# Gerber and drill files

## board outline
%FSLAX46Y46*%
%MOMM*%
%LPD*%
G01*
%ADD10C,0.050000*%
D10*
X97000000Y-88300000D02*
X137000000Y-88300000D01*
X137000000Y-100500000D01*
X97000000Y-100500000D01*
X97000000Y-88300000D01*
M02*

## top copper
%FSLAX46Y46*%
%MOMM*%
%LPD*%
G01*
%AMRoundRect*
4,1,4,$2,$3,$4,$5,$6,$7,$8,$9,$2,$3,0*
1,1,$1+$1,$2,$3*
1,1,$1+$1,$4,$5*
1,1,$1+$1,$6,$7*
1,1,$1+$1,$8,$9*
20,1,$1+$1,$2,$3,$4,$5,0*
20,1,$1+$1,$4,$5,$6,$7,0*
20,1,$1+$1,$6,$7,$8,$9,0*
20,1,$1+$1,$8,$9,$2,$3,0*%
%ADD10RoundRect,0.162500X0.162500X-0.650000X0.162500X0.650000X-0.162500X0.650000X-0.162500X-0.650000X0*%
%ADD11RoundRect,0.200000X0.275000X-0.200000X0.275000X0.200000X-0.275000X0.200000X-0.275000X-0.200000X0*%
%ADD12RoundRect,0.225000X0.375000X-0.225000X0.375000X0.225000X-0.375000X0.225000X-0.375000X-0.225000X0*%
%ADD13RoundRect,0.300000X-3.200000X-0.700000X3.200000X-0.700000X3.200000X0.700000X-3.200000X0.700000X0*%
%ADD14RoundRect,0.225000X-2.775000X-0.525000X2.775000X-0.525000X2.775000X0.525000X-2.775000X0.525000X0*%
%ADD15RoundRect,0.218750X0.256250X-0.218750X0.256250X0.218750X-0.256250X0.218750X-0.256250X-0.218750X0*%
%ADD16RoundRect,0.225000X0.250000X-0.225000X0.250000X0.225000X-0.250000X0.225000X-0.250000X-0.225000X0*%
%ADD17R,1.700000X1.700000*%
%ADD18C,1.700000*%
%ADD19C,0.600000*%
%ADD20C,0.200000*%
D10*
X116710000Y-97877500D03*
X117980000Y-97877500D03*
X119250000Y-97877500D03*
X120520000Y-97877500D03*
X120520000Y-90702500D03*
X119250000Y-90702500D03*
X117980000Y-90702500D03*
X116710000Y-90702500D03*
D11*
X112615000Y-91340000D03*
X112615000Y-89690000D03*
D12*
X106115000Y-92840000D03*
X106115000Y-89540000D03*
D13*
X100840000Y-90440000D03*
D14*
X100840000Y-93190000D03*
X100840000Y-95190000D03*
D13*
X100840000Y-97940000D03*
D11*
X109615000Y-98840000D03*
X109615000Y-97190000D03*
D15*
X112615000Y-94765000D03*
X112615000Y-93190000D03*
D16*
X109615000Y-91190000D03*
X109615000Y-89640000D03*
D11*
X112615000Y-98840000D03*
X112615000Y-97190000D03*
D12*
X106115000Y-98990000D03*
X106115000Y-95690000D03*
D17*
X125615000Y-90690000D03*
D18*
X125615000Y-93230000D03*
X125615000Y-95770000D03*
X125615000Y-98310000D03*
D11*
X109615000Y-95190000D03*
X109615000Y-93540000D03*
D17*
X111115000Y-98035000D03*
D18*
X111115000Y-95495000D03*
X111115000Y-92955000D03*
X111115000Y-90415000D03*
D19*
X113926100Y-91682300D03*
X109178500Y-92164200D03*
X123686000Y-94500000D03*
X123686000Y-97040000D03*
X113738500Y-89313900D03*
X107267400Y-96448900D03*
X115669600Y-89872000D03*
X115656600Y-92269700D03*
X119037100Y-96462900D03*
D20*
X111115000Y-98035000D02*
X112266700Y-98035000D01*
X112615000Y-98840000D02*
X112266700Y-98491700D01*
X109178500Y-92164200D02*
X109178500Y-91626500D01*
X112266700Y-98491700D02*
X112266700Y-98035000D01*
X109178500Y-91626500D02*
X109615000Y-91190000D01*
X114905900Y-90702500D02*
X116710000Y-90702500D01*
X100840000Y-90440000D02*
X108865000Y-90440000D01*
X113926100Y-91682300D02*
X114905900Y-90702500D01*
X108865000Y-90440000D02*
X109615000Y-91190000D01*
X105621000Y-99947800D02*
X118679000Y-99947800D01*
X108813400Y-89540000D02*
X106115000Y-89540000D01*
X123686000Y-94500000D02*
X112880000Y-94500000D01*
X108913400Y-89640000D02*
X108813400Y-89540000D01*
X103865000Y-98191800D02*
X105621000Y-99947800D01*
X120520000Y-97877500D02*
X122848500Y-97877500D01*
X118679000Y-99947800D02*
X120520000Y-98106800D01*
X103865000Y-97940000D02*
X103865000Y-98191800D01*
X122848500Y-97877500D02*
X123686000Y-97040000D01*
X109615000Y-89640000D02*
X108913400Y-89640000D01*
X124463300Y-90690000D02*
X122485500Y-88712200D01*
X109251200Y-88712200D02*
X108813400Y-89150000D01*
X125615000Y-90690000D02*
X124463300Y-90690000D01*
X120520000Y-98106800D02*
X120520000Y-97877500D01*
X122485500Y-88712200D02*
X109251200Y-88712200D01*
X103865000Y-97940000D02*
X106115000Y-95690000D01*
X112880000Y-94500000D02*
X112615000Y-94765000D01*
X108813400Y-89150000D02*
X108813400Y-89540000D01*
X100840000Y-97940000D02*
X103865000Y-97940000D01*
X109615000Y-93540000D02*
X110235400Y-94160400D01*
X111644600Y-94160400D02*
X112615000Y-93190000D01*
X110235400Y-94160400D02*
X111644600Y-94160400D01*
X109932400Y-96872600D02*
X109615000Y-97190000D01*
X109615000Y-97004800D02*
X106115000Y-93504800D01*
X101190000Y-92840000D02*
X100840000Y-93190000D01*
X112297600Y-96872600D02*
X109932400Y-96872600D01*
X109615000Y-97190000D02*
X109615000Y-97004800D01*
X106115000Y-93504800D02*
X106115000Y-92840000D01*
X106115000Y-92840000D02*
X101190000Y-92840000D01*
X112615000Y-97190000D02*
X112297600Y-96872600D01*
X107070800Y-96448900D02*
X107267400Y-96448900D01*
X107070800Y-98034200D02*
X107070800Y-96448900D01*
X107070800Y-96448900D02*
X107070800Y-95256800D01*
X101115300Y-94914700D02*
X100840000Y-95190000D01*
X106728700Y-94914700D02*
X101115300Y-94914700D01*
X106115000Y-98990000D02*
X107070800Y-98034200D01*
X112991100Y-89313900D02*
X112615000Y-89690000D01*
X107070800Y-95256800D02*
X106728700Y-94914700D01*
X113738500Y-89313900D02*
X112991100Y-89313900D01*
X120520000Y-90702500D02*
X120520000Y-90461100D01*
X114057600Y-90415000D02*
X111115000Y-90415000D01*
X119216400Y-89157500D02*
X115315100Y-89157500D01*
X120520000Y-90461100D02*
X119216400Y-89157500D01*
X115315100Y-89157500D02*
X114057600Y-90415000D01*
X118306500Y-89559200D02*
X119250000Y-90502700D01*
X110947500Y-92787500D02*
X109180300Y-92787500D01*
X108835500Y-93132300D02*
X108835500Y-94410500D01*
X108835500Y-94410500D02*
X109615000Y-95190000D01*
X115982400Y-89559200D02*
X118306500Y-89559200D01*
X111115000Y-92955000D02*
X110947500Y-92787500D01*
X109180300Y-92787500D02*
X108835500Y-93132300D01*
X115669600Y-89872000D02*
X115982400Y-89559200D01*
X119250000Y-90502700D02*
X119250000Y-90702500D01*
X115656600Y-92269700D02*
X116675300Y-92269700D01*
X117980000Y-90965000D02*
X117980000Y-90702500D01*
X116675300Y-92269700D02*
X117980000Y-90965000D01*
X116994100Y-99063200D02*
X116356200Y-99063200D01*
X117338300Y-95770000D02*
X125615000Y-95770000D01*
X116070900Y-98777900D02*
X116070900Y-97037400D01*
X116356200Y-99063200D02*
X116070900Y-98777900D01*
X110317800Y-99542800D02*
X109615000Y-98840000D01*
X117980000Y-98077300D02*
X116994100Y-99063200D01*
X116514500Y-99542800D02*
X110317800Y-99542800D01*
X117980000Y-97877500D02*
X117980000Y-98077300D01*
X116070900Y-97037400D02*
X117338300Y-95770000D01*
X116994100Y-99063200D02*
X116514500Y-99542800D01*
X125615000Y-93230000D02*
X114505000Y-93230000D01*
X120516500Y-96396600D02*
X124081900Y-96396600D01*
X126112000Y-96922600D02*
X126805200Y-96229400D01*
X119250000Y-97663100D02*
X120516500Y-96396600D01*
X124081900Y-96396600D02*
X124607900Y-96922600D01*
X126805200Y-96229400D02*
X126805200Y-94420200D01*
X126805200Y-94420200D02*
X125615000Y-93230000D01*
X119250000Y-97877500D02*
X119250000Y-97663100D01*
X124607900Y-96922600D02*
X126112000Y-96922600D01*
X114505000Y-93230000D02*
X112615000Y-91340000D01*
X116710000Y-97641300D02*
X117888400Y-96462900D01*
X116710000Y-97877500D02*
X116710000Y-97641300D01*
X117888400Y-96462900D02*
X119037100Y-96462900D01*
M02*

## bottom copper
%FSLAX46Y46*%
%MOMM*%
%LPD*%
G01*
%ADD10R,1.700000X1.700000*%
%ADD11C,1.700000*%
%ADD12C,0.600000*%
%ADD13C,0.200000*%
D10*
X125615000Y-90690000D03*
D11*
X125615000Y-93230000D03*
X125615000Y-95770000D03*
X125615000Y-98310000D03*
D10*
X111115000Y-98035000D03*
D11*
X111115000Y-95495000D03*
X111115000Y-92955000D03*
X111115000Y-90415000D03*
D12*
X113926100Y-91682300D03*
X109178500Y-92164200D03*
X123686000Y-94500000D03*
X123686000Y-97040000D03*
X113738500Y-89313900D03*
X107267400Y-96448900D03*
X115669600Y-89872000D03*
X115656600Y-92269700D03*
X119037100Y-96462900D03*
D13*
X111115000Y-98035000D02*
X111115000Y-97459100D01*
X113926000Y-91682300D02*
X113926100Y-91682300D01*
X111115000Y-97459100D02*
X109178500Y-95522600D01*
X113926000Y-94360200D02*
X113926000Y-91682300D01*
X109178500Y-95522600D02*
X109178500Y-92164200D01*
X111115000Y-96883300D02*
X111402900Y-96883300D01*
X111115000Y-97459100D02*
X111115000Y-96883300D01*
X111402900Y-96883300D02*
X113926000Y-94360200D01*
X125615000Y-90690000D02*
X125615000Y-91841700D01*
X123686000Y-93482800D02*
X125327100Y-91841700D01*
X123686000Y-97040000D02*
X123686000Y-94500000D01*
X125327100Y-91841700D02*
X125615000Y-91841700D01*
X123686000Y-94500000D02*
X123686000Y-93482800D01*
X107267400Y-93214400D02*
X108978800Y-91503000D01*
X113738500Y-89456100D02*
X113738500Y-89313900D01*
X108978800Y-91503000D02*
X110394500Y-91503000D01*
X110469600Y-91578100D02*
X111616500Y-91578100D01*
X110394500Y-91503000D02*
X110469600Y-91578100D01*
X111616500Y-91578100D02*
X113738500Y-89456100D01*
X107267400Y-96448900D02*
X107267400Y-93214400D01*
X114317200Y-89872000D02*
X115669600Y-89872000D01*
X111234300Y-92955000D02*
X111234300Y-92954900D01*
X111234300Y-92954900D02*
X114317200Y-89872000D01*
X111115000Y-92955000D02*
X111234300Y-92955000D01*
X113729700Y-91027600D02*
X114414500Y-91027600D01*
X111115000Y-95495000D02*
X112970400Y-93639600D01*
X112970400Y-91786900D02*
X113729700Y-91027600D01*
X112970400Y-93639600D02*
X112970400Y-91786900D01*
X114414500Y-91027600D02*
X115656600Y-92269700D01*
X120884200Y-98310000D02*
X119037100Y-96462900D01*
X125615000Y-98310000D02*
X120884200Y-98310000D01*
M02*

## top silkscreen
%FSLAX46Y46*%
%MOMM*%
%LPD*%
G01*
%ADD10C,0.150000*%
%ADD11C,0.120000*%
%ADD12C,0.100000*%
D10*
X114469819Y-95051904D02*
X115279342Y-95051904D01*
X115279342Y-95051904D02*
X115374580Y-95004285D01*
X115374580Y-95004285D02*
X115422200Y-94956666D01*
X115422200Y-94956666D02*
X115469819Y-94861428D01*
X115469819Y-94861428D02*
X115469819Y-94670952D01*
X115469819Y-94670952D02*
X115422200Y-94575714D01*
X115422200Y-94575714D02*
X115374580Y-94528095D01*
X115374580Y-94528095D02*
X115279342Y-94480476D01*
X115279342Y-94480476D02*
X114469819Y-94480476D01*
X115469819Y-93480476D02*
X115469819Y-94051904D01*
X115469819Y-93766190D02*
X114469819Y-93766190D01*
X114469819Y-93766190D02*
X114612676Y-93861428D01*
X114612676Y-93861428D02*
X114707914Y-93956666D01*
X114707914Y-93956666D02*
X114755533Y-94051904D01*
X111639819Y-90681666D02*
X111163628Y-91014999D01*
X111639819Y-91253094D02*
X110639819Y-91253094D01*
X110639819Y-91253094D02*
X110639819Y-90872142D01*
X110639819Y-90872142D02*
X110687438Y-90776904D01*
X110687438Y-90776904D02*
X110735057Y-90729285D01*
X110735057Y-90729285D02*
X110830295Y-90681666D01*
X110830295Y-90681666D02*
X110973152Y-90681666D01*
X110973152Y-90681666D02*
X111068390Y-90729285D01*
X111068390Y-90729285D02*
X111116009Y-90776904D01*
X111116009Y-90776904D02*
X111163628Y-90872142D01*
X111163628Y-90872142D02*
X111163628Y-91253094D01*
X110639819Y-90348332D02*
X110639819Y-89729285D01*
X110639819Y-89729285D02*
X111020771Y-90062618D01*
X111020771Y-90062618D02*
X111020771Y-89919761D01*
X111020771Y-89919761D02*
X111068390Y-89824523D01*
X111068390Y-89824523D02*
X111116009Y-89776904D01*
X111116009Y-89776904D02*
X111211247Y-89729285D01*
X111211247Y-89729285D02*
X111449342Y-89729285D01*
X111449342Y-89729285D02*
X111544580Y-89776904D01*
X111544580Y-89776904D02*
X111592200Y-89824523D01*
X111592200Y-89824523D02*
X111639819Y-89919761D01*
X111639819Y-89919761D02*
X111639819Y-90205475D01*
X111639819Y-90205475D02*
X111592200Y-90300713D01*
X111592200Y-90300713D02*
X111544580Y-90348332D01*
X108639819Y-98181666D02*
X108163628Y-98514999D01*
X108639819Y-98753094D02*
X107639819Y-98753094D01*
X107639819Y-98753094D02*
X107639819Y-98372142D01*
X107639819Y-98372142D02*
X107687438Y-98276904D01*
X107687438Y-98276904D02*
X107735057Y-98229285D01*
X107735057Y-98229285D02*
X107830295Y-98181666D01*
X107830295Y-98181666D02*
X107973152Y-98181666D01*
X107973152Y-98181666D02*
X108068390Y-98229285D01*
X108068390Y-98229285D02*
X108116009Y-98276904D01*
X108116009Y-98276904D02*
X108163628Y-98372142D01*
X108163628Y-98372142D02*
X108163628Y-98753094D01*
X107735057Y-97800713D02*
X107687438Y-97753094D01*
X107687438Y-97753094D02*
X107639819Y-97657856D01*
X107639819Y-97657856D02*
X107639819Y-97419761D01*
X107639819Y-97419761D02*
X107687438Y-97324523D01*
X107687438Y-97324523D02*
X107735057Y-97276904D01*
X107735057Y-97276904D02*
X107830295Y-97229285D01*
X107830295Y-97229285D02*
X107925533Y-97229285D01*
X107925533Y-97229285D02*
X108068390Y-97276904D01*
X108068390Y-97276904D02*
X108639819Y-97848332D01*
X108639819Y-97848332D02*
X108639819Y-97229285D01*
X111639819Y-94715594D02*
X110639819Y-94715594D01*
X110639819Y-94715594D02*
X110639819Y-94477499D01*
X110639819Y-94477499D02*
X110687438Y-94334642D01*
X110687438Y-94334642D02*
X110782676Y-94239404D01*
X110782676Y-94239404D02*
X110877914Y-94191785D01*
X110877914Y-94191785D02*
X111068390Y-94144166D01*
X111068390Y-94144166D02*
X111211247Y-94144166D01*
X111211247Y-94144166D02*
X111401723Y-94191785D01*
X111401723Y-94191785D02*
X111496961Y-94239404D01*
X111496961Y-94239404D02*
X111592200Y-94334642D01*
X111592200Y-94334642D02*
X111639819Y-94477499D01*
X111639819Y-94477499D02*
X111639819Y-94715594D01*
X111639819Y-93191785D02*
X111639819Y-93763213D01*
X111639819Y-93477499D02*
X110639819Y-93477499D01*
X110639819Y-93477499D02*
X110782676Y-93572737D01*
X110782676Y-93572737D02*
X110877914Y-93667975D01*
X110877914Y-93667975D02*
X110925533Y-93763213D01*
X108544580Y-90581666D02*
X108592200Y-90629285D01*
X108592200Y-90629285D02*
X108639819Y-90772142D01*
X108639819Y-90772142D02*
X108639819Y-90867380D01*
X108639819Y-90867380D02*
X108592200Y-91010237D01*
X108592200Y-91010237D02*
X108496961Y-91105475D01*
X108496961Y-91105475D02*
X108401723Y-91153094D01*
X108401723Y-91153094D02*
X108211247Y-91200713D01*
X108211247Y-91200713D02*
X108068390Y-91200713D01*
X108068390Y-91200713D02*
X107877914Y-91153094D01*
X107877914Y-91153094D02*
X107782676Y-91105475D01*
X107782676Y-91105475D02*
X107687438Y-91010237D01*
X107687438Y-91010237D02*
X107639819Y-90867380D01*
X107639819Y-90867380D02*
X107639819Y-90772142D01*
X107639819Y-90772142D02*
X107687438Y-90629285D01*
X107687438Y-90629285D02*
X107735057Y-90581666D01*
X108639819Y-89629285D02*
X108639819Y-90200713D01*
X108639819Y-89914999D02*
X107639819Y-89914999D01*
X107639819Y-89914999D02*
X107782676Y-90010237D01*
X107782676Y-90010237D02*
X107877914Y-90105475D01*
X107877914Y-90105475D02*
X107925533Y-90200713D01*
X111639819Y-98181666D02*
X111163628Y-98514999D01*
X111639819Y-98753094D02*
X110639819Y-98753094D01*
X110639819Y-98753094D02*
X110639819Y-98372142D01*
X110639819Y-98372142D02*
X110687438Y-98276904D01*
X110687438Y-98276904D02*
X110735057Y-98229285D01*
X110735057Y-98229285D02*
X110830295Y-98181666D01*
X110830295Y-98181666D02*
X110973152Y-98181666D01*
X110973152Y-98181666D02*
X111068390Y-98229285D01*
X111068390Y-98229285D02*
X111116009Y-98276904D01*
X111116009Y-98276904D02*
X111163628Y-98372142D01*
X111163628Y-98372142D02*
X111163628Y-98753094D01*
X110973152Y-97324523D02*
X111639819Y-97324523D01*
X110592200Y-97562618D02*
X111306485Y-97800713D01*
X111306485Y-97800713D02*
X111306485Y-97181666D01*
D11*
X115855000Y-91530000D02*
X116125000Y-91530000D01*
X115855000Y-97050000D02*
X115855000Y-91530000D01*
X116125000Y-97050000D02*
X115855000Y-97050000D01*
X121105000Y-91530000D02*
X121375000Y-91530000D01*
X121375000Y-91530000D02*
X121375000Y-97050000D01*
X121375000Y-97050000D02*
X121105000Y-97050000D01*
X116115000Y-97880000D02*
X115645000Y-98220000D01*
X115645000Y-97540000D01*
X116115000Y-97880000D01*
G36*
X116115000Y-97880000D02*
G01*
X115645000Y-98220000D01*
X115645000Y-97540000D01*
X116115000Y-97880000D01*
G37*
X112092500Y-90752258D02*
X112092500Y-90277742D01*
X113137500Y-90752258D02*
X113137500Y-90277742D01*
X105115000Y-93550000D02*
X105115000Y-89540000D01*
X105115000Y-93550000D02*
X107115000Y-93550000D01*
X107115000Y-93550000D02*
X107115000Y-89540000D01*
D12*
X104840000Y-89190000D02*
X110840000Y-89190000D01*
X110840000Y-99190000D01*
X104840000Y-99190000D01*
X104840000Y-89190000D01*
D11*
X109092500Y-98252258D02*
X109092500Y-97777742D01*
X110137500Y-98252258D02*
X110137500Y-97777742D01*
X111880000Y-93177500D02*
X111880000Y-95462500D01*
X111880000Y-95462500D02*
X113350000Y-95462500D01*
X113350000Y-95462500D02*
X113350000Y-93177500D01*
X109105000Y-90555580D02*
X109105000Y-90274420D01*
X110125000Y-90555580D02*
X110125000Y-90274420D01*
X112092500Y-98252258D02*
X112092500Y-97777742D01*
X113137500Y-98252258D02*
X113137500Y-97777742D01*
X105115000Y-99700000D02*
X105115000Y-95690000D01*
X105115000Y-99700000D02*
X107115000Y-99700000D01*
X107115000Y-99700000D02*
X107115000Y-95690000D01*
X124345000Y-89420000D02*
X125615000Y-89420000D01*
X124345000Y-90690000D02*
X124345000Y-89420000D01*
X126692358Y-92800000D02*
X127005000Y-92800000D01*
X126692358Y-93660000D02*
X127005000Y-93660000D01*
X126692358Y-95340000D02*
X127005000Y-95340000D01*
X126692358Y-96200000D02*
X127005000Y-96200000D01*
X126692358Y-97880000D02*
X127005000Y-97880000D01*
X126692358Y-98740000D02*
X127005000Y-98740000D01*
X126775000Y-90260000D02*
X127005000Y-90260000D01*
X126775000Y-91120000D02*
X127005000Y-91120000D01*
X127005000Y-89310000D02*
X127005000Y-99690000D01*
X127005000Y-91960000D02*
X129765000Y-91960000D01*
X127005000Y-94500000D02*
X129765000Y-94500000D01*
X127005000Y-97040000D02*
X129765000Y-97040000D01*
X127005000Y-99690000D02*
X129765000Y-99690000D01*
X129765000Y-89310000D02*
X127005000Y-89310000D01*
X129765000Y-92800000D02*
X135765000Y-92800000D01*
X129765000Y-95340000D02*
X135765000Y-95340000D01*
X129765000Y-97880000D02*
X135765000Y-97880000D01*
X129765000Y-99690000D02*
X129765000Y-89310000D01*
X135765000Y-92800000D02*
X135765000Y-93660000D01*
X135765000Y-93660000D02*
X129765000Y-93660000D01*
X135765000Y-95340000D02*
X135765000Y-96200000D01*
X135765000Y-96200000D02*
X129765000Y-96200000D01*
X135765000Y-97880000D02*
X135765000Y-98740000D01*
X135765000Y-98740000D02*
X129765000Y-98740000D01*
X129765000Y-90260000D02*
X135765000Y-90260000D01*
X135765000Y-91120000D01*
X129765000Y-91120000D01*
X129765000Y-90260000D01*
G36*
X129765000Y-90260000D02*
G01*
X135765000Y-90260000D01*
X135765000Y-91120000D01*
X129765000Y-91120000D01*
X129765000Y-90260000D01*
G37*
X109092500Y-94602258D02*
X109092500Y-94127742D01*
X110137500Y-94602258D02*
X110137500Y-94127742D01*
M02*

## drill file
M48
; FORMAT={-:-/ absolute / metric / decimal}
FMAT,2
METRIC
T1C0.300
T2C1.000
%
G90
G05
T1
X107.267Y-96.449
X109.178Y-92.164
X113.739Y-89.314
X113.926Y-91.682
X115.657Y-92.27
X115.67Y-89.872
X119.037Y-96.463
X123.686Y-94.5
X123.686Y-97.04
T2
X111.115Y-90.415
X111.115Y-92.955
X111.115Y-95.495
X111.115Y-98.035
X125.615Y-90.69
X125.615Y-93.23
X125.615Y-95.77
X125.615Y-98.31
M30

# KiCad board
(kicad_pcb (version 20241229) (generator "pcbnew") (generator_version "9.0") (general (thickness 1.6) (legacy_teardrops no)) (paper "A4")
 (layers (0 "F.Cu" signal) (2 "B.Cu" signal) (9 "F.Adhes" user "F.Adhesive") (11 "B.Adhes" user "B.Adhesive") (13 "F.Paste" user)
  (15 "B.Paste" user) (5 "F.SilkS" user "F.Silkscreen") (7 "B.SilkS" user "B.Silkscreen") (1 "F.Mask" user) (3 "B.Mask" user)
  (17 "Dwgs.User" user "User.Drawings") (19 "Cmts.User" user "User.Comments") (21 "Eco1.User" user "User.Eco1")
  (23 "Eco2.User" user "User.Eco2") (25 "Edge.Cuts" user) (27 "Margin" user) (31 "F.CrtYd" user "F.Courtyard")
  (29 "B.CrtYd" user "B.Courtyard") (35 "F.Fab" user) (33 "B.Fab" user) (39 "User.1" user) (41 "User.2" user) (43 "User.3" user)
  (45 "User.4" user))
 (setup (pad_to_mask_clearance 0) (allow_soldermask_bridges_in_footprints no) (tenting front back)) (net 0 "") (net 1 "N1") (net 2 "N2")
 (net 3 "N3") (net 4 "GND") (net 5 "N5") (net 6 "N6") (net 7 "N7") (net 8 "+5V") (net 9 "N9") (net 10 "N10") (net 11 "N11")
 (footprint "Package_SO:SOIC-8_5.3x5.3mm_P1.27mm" (layer "F.Cu") (at 118.615 94.29 90)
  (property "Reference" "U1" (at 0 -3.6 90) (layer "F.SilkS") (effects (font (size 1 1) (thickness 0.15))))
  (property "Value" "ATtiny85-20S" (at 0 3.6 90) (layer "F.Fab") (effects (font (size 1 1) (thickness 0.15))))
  (fp_line (start 2.76 -2.76) (end 2.76 -2.49) (stroke (width 0.12) (type solid)) (layer "F.SilkS"))
  (fp_line (start -2.76 -2.76) (end 2.76 -2.76) (stroke (width 0.12) (type solid)) (layer "F.SilkS"))
  (fp_line (start -2.76 -2.49) (end -2.76 -2.76) (stroke (width 0.12) (type solid)) (layer "F.SilkS"))
  (fp_line (start 2.76 2.49) (end 2.76 2.76) (stroke (width 0.12) (type solid)) (layer "F.SilkS"))
  (fp_line (start 2.76 2.76) (end -2.76 2.76) (stroke (width 0.12) (type solid)) (layer "F.SilkS"))
  (fp_line (start -2.76 2.76) (end -2.76 2.49) (stroke (width 0.12) (type solid)) (layer "F.SilkS"))
  (fp_poly (pts (xy -3.59 -2.5) (xy -3.93 -2.97) (xy -3.25 -2.97)) (stroke (width 0.12) (type solid)) (fill yes) (layer "F.SilkS"))
  (pad "1" smd roundrect (at -3.5875 -1.905 90) (size 1.625 0.65) (layers "F.Cu" "F.Mask" "F.Paste") (roundrect_rratio 0.25) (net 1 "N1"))
  (pad "2" smd roundrect (at -3.5875 -0.635 90) (size 1.625 0.65) (layers "F.Cu" "F.Mask" "F.Paste") (roundrect_rratio 0.25) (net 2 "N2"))
  (pad "3" smd roundrect (at -3.5875 0.635 90) (size 1.625 0.65) (layers "F.Cu" "F.Mask" "F.Paste") (roundrect_rratio 0.25) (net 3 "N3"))
  (pad "4" smd roundrect (at -3.5875 1.905 90) (size 1.625 0.65) (layers "F.Cu" "F.Mask" "F.Paste") (roundrect_rratio 0.25) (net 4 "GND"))
  (pad "5" smd roundrect (at 3.5875 1.905 90) (size 1.625 0.65) (layers "F.Cu" "F.Mask" "F.Paste") (roundrect_rratio 0.25) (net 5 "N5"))
  (pad "6" smd roundrect (at 3.5875 0.635 90) (size 1.625 0.65) (layers "F.Cu" "F.Mask" "F.Paste") (roundrect_rratio 0.25) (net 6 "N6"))
  (pad "7" smd roundrect (at 3.5875 -0.635 90) (size 1.625 0.65) (layers "F.Cu" "F.Mask" "F.Paste") (roundrect_rratio 0.25) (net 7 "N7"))
  (pad "8" smd roundrect (at 3.5875 -1.905 90) (size 1.625 0.65) (layers "F.Cu" "F.Mask" "F.Paste") (roundrect_rratio 0.25) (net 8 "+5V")))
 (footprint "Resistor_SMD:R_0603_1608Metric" (layer "F.Cu") (at 112.615 90.515 90)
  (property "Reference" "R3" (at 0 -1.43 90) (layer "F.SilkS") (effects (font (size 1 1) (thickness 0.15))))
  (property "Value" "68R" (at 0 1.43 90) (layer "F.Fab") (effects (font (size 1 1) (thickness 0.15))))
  (fp_line (start -0.237258 -0.5225) (end 0.237258 -0.5225) (stroke (width 0.12) (type solid)) (layer "F.SilkS"))
  (fp_line (start -0.237258 0.5225) (end 0.237258 0.5225) (stroke (width 0.12) (type solid)) (layer "F.SilkS"))
  (pad "1" smd roundrect (at -0.825 0 90) (size 0.8 0.95) (layers "F.Cu" "F.Mask" "F.Paste") (roundrect_rratio 0.25) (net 3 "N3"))
  (pad "2" smd roundrect (at 0.825 0 90) (size 0.8 0.95) (layers "F.Cu" "F.Mask" "F.Paste") (roundrect_rratio 0.25) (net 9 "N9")))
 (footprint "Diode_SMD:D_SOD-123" (layer "F.Cu") (at 106.115 91.19 90)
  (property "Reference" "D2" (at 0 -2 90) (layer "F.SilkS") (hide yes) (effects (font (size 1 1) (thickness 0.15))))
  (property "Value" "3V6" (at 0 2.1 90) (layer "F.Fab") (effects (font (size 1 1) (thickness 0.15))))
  (fp_line (start -2.36 -1) (end 1.65 -1) (stroke (width 0.12) (type solid)) (layer "F.SilkS"))
  (fp_line (start -2.36 -1) (end -2.36 1) (stroke (width 0.12) (type solid)) (layer "F.SilkS"))
  (fp_line (start -2.36 1) (end 1.65 1) (stroke (width 0.12) (type solid)) (layer "F.SilkS"))
  (pad "1" smd roundrect (at -1.65 0 90) (size 0.9 1.2) (layers "F.Cu" "F.Mask" "F.Paste") (roundrect_rratio 0.25) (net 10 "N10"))
  (pad "2" smd roundrect (at 1.65 0 90) (size 0.9 1.2) (layers "F.Cu" "F.Mask" "F.Paste") (roundrect_rratio 0.25) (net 4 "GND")))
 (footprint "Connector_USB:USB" (layer "F.Cu") (at 100.84 94.19)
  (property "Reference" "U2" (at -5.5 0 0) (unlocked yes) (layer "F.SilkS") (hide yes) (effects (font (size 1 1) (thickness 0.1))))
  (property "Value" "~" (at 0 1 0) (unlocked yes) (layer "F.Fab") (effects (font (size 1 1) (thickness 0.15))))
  (fp_rect (start 4 -5) (end 10 5) (stroke (width 0.1) (type default)) (fill no) (layer "F.SilkS"))
  (pad "1" smd roundrect (at 0 -3.75) (size 7 2) (layers "F.Cu" "F.Mask" "F.Paste") (roundrect_rratio 0.15) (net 8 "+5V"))
  (pad "2" smd roundrect (at 0 -1) (size 6 1.5) (layers "F.Cu" "F.Mask" "F.Paste") (roundrect_rratio 0.15) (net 10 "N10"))
  (pad "3" smd roundrect (at 0 1) (size 6 1.5) (layers "F.Cu" "F.Mask" "F.Paste") (roundrect_rratio 0.15) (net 9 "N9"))
  (pad "4" smd roundrect (at 0 3.75) (size 7 2) (layers "F.Cu" "F.Mask" "F.Paste") (roundrect_rratio 0.15) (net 4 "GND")))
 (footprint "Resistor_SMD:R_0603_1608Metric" (layer "F.Cu") (at 109.615 98.015 90)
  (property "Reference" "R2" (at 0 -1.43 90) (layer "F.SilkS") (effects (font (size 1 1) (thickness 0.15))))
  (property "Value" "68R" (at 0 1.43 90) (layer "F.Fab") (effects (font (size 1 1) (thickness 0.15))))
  (fp_line (start -0.237258 -0.5225) (end 0.237258 -0.5225) (stroke (width 0.12) (type solid)) (layer "F.SilkS"))
  (fp_line (start -0.237258 0.5225) (end 0.237258 0.5225) (stroke (width 0.12) (type solid)) (layer "F.SilkS"))
  (pad "1" smd roundrect (at -0.825 0 90) (size 0.8 0.95) (layers "F.Cu" "F.Mask" "F.Paste") (roundrect_rratio 0.25) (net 2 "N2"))
  (pad "2" smd roundrect (at 0.825 0 90) (size 0.8 0.95) (layers "F.Cu" "F.Mask" "F.Paste") (roundrect_rratio 0.25) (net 10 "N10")))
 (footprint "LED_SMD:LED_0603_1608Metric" (layer "F.Cu") (at 112.615 93.9775 90)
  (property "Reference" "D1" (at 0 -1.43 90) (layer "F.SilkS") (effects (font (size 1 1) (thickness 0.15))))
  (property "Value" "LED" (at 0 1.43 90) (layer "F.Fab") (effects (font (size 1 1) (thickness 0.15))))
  (fp_line (start 0.8 -0.735) (end -1.485 -0.735) (stroke (width 0.12) (type solid)) (layer "F.SilkS"))
  (fp_line (start -1.485 -0.735) (end -1.485 0.735) (stroke (width 0.12) (type solid)) (layer "F.SilkS"))
  (fp_line (start -1.485 0.735) (end 0.8 0.735) (stroke (width 0.12) (type solid)) (layer "F.SilkS"))
  (pad "1" smd roundrect (at -0.7875 0 90) (size 0.875 0.95) (layers "F.Cu" "F.Mask" "F.Paste") (roundrect_rratio 0.25) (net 4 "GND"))
  (pad "2" smd roundrect (at 0.7875 0 90) (size 0.875 0.95) (layers "F.Cu" "F.Mask" "F.Paste") (roundrect_rratio 0.25) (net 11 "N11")))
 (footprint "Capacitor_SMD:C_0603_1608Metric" (layer "F.Cu") (at 109.615 90.415 90)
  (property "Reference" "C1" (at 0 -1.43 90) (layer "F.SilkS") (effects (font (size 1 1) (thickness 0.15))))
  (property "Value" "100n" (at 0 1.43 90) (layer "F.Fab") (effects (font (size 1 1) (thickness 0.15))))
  (fp_line (start -0.14058 -0.51) (end 0.14058 -0.51) (stroke (width 0.12) (type solid)) (layer "F.SilkS"))
  (fp_line (start -0.14058 0.51) (end 0.14058 0.51) (stroke (width 0.12) (type solid)) (layer "F.SilkS"))
  (pad "1" smd roundrect (at -0.775 0 90) (size 0.9 0.95) (layers "F.Cu" "F.Mask" "F.Paste") (roundrect_rratio 0.25) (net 8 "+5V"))
  (pad "2" smd roundrect (at 0.775 0 90) (size 0.9 0.95) (layers "F.Cu" "F.Mask" "F.Paste") (roundrect_rratio 0.25) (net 4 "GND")))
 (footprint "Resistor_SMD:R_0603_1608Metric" (layer "F.Cu") (at 112.615 98.015 90)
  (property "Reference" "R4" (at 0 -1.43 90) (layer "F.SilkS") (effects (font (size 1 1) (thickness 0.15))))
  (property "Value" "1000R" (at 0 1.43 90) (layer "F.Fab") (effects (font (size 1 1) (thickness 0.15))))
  (fp_line (start -0.237258 -0.5225) (end 0.237258 -0.5225) (stroke (width 0.12) (type solid)) (layer "F.SilkS"))
  (fp_line (start -0.237258 0.5225) (end 0.237258 0.5225) (stroke (width 0.12) (type solid)) (layer "F.SilkS"))
  (pad "1" smd roundrect (at -0.825 0 90) (size 0.8 0.95) (layers "F.Cu" "F.Mask" "F.Paste") (roundrect_rratio 0.25) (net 8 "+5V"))
  (pad "2" smd roundrect (at 0.825 0 90) (size 0.8 0.95) (layers "F.Cu" "F.Mask" "F.Paste") (roundrect_rratio 0.25) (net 10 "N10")))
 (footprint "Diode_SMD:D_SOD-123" (layer "F.Cu") (at 106.115 97.34 90)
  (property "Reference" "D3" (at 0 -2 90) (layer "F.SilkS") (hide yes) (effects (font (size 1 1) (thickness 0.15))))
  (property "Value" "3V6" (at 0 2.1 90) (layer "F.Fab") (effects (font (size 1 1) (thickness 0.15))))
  (fp_line (start -2.36 -1) (end 1.65 -1) (stroke (width 0.12) (type solid)) (layer "F.SilkS"))
  (fp_line (start -2.36 -1) (end -2.36 1) (stroke (width 0.12) (type solid)) (layer "F.SilkS"))
  (fp_line (start -2.36 1) (end 1.65 1) (stroke (width 0.12) (type solid)) (layer "F.SilkS"))
  (pad "1" smd roundrect (at -1.65 0 90) (size 0.9 1.2) (layers "F.Cu" "F.Mask" "F.Paste") (roundrect_rratio 0.25) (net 9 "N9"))
  (pad "2" smd roundrect (at 1.65 0 90) (size 0.9 1.2) (layers "F.Cu" "F.Mask" "F.Paste") (roundrect_rratio 0.25) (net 4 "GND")))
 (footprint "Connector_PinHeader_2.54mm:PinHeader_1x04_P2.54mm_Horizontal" (layer "F.Cu") (at 125.615 90.69)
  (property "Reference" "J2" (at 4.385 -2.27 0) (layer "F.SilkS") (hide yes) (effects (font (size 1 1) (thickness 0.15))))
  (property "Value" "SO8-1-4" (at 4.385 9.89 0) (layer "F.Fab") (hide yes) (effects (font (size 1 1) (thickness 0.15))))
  (fp_line (start -1.27 -1.27) (end 0 -1.27) (stroke (width 0.12) (type solid)) (layer "F.SilkS"))
  (fp_line (start -1.27 0) (end -1.27 -1.27) (stroke (width 0.12) (type solid)) (layer "F.SilkS"))
  (fp_line (start 1.077358 2.11) (end 1.39 2.11) (stroke (width 0.12) (type solid)) (layer "F.SilkS"))
  (fp_line (start 1.077358 2.97) (end 1.39 2.97) (stroke (width 0.12) (type solid)) (layer "F.SilkS"))
  (fp_line (start 1.077358 4.65) (end 1.39 4.65) (stroke (width 0.12) (type solid)) (layer "F.SilkS"))
  (fp_line (start 1.077358 5.51) (end 1.39 5.51) (stroke (width 0.12) (type solid)) (layer "F.SilkS"))
  (fp_line (start 1.077358 7.19) (end 1.39 7.19) (stroke (width 0.12) (type solid)) (layer "F.SilkS"))
  (fp_line (start 1.077358 8.05) (end 1.39 8.05) (stroke (width 0.12) (type solid)) (layer "F.SilkS"))
  (fp_line (start 1.16 -0.43) (end 1.39 -0.43) (stroke (width 0.12) (type solid)) (layer "F.SilkS"))
  (fp_line (start 1.16 0.43) (end 1.39 0.43) (stroke (width 0.12) (type solid)) (layer "F.SilkS"))
  (fp_line (start 1.39 -1.38) (end 1.39 9) (stroke (width 0.12) (type solid)) (layer "F.SilkS"))
  (fp_line (start 1.39 1.27) (end 4.15 1.27) (stroke (width 0.12) (type solid)) (layer "F.SilkS"))
  (fp_line (start 1.39 3.81) (end 4.15 3.81) (stroke (width 0.12) (type solid)) (layer "F.SilkS"))
  (fp_line (start 1.39 6.35) (end 4.15 6.35) (stroke (width 0.12) (type solid)) (layer "F.SilkS"))
  (fp_line (start 1.39 9) (end 4.15 9) (stroke (width 0.12) (type solid)) (layer "F.SilkS"))
  (fp_line (start 4.15 -1.38) (end 1.39 -1.38) (stroke (width 0.12) (type solid)) (layer "F.SilkS"))
  (fp_line (start 4.15 2.11) (end 10.15 2.11) (stroke (width 0.12) (type solid)) (layer "F.SilkS"))
  (fp_line (start 4.15 4.65) (end 10.15 4.65) (stroke (width 0.12) (type solid)) (layer "F.SilkS"))
  (fp_line (start 4.15 7.19) (end 10.15 7.19) (stroke (width 0.12) (type solid)) (layer "F.SilkS"))
  (fp_line (start 4.15 9) (end 4.15 -1.38) (stroke (width 0.12) (type solid)) (layer "F.SilkS"))
  (fp_line (start 10.15 2.11) (end 10.15 2.97) (stroke (width 0.12) (type solid)) (layer "F.SilkS"))
  (fp_line (start 10.15 2.97) (end 4.15 2.97) (stroke (width 0.12) (type solid)) (layer "F.SilkS"))
  (fp_line (start 10.15 4.65) (end 10.15 5.51) (stroke (width 0.12) (type solid)) (layer "F.SilkS"))
  (fp_line (start 10.15 5.51) (end 4.15 5.51) (stroke (width 0.12) (type solid)) (layer "F.SilkS"))
  (fp_line (start 10.15 7.19) (end 10.15 8.05) (stroke (width 0.12) (type solid)) (layer "F.SilkS"))
  (fp_line (start 10.15 8.05) (end 4.15 8.05) (stroke (width 0.12) (type solid)) (layer "F.SilkS"))
  (fp_rect (start 4.15 -0.43) (end 10.15 0.43) (stroke (width 0.12) (type solid)) (fill yes) (layer "F.SilkS"))
  (pad "1" thru_hole rect (at 0 0) (size 1.7 1.7) (drill 1) (layers "*.Cu" "*.Mask") (remove_unused_layers no) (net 4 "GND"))
  (pad "2" thru_hole circle (at 0 2.54) (size 1.7 1.7) (drill 1) (layers "*.Cu" "*.Mask") (remove_unused_layers no) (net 3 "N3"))
  (pad "3" thru_hole circle (at 0 5.08) (size 1.7 1.7) (drill 1) (layers "*.Cu" "*.Mask") (remove_unused_layers no) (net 2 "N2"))
  (pad "4" thru_hole circle (at 0 7.62) (size 1.7 1.7) (drill 1) (layers "*.Cu" "*.Mask") (remove_unused_layers no) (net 1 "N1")))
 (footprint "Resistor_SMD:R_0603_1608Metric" (layer "F.Cu") (at 109.615 94.365 90)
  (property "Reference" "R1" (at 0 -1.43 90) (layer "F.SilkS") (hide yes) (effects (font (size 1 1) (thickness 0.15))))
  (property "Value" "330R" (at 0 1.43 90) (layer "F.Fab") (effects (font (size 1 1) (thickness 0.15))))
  (fp_line (start -0.237258 -0.5225) (end 0.237258 -0.5225) (stroke (width 0.12) (type solid)) (layer "F.SilkS"))
  (fp_line (start -0.237258 0.5225) (end 0.237258 0.5225) (stroke (width 0.12) (type solid)) (layer "F.SilkS"))
  (pad "1" smd roundrect (at -0.825 0 90) (size 0.8 0.95) (layers "F.Cu" "F.Mask" "F.Paste") (roundrect_rratio 0.25) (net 6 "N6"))
  (pad "2" smd roundrect (at 0.825 0 90) (size 0.8 0.95) (layers "F.Cu" "F.Mask" "F.Paste") (roundrect_rratio 0.25) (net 11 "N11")))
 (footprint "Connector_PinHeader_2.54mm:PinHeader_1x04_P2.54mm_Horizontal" (layer "B.Cu") (at 111.115 98.035)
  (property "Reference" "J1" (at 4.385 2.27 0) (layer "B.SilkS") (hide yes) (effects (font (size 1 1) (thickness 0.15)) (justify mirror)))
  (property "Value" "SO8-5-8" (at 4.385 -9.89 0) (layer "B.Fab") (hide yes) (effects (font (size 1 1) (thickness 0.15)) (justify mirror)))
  (pad "1" thru_hole rect (at 0 0) (size 1.7 1.7) (drill 1) (layers "*.Cu" "*.Mask") (remove_unused_layers no) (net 8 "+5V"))
  (pad "2" thru_hole circle (at 0 -2.54) (size 1.7 1.7) (drill 1) (layers "*.Cu" "*.Mask") (remove_unused_layers no) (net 7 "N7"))
  (pad "3" thru_hole circle (at 0 -5.08) (size 1.7 1.7) (drill 1) (layers "*.Cu" "*.Mask") (remove_unused_layers no) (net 6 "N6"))
  (pad "4" thru_hole circle (at 0 -7.62) (size 1.7 1.7) (drill 1) (layers "*.Cu" "*.Mask") (remove_unused_layers no) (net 5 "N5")))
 (gr_rect (start 97 88.3) (end 137 100.5) (stroke (width 0.05) (type solid)) (fill no) (layer "Edge.Cuts"))
 (segment (start 111.115 98.035) (end 112.2667 98.035) (width 0.2) (layer "F.Cu") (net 8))
 (segment (start 112.615 98.84) (end 112.2667 98.4917) (width 0.2) (layer "F.Cu") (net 8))
 (segment (start 109.1785 92.1642) (end 109.1785 91.6265) (width 0.2) (layer "F.Cu") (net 8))
 (segment (start 112.2667 98.4917) (end 112.2667 98.035) (width 0.2) (layer "F.Cu") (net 8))
 (segment (start 109.1785 91.6265) (end 109.615 91.19) (width 0.2) (layer "F.Cu") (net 8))
 (segment (start 114.9059 90.7025) (end 116.71 90.7025) (width 0.2) (layer "F.Cu") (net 8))
 (segment (start 100.84 90.44) (end 108.865 90.44) (width 0.2) (layer "F.Cu") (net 8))
 (segment (start 113.9261 91.6823) (end 114.9059 90.7025) (width 0.2) (layer "F.Cu") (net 8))
 (segment (start 108.865 90.44) (end 109.615 91.19) (width 0.2) (layer "F.Cu") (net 8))
 (via (at 113.9261 91.6823) (size 0.6) (drill 0.3) (layers "F.Cu" "B.Cu") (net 8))
 (via (at 109.1785 92.1642) (size 0.6) (drill 0.3) (layers "F.Cu" "B.Cu") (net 8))
 (segment (start 111.115 98.035) (end 111.115 97.4591) (width 0.2) (layer "B.Cu") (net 8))
 (segment (start 113.926 91.6823) (end 113.9261 91.6823) (width 0.2) (layer "B.Cu") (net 8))
 (segment (start 111.115 97.4591) (end 109.1785 95.5226) (width 0.2) (layer "B.Cu") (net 8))
 (segment (start 113.926 94.3602) (end 113.926 91.6823) (width 0.2) (layer "B.Cu") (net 8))
 (segment (start 109.1785 95.5226) (end 109.1785 92.1642) (width 0.2) (layer "B.Cu") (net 8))
 (segment (start 111.115 96.8833) (end 111.4029 96.8833) (width 0.2) (layer "B.Cu") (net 8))
 (segment (start 111.115 97.4591) (end 111.115 96.8833) (width 0.2) (layer "B.Cu") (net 8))
 (segment (start 111.4029 96.8833) (end 113.926 94.3602) (width 0.2) (layer "B.Cu") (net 8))
 (segment (start 105.621 99.9478) (end 118.679 99.9478) (width 0.2) (layer "F.Cu") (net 4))
 (segment (start 108.8134 89.54) (end 106.115 89.54) (width 0.2) (layer "F.Cu") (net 4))
 (segment (start 123.686 94.5) (end 112.88 94.5) (width 0.2) (layer "F.Cu") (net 4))
 (segment (start 108.9134 89.64) (end 108.8134 89.54) (width 0.2) (layer "F.Cu") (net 4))
 (segment (start 103.865 98.1918) (end 105.621 99.9478) (width 0.2) (layer "F.Cu") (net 4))
 (segment (start 120.52 97.8775) (end 122.8485 97.8775) (width 0.2) (layer "F.Cu") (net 4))
 (segment (start 118.679 99.9478) (end 120.52 98.1068) (width 0.2) (layer "F.Cu") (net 4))
 (segment (start 103.865 97.94) (end 103.865 98.1918) (width 0.2) (layer "F.Cu") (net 4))
 (segment (start 122.8485 97.8775) (end 123.686 97.04) (width 0.2) (layer "F.Cu") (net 4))
 (segment (start 109.615 89.64) (end 108.9134 89.64) (width 0.2) (layer "F.Cu") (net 4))
 (segment (start 124.4633 90.69) (end 122.4855 88.7122) (width 0.2) (layer "F.Cu") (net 4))
 (segment (start 109.2512 88.7122) (end 108.8134 89.15) (width 0.2) (layer "F.Cu") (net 4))
 (segment (start 125.615 90.69) (end 124.4633 90.69) (width 0.2) (layer "F.Cu") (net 4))
 (segment (start 120.52 98.1068) (end 120.52 97.8775) (width 0.2) (layer "F.Cu") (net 4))
 (segment (start 122.4855 88.7122) (end 109.2512 88.7122) (width 0.2) (layer "F.Cu") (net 4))
 (segment (start 103.865 97.94) (end 106.115 95.69) (width 0.2) (layer "F.Cu") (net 4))
 (segment (start 112.88 94.5) (end 112.615 94.765) (width 0.2) (layer "F.Cu") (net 4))
 (segment (start 108.8134 89.15) (end 108.8134 89.54) (width 0.2) (layer "F.Cu") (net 4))
 (segment (start 100.84 97.94) (end 103.865 97.94) (width 0.2) (layer "F.Cu") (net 4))
 (via (at 123.686 94.5) (size 0.6) (drill 0.3) (layers "F.Cu" "B.Cu") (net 4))
 (via (at 123.686 97.04) (size 0.6) (drill 0.3) (layers "F.Cu" "B.Cu") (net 4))
 (segment (start 125.615 90.69) (end 125.615 91.8417) (width 0.2) (layer "B.Cu") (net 4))
 (segment (start 123.686 93.4828) (end 125.3271 91.8417) (width 0.2) (layer "B.Cu") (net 4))
 (segment (start 123.686 97.04) (end 123.686 94.5) (width 0.2) (layer "B.Cu") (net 4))
 (segment (start 125.3271 91.8417) (end 125.615 91.8417) (width 0.2) (layer "B.Cu") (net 4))
 (segment (start 123.686 94.5) (end 123.686 93.4828) (width 0.2) (layer "B.Cu") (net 4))
 (segment (start 109.615 93.54) (end 110.2354 94.1604) (width 0.2) (layer "F.Cu") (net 11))
 (segment (start 111.6446 94.1604) (end 112.615 93.19) (width 0.2) (layer "F.Cu") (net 11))
 (segment (start 110.2354 94.1604) (end 111.6446 94.1604) (width 0.2) (layer "F.Cu") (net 11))
 (segment (start 109.9324 96.8726) (end 109.615 97.19) (width 0.2) (layer "F.Cu") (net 10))
 (segment (start 109.615 97.0048) (end 106.115 93.5048) (width 0.2) (layer "F.Cu") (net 10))
 (segment (start 101.19 92.84) (end 100.84 93.19) (width 0.2) (layer "F.Cu") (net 10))
 (segment (start 112.2976 96.8726) (end 109.9324 96.8726) (width 0.2) (layer "F.Cu") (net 10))
 (segment (start 109.615 97.19) (end 109.615 97.0048) (width 0.2) (layer "F.Cu") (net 10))
 (segment (start 106.115 93.5048) (end 106.115 92.84) (width 0.2) (layer "F.Cu") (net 10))
 (segment (start 106.115 92.84) (end 101.19 92.84) (width 0.2) (layer "F.Cu") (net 10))
 (segment (start 112.615 97.19) (end 112.2976 96.8726) (width 0.2) (layer "F.Cu") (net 10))
 (segment (start 107.0708 96.4489) (end 107.2674 96.4489) (width 0.2) (layer "F.Cu") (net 9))
 (segment (start 107.0708 98.0342) (end 107.0708 96.4489) (width 0.2) (layer "F.Cu") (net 9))
 (segment (start 107.0708 96.4489) (end 107.0708 95.2568) (width 0.2) (layer "F.Cu") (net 9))
 (segment (start 101.1153 94.9147) (end 100.84 95.19) (width 0.2) (layer "F.Cu") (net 9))
 (segment (start 106.7287 94.9147) (end 101.1153 94.9147) (width 0.2) (layer "F.Cu") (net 9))
 (segment (start 106.115 98.99) (end 107.0708 98.0342) (width 0.2) (layer "F.Cu") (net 9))
 (segment (start 112.9911 89.3139) (end 112.615 89.69) (width 0.2) (layer "F.Cu") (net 9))
 (segment (start 107.0708 95.2568) (end 106.7287 94.9147) (width 0.2) (layer "F.Cu") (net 9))
 (segment (start 113.7385 89.3139) (end 112.9911 89.3139) (width 0.2) (layer "F.Cu") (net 9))
 (via (at 113.7385 89.3139) (size 0.6) (drill 0.3) (layers "F.Cu" "B.Cu") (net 9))
 (via (at 107.2674 96.4489) (size 0.6) (drill 0.3) (layers "F.Cu" "B.Cu") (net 9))
 (segment (start 107.2674 93.2144) (end 108.9788 91.503) (width 0.2) (layer "B.Cu") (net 9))
 (segment (start 113.7385 89.4561) (end 113.7385 89.3139) (width 0.2) (layer "B.Cu") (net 9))
 (segment (start 108.9788 91.503) (end 110.3945 91.503) (width 0.2) (layer "B.Cu") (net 9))
 (segment (start 110.4696 91.5781) (end 111.6165 91.5781) (width 0.2) (layer "B.Cu") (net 9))
 (segment (start 110.3945 91.503) (end 110.4696 91.5781) (width 0.2) (layer "B.Cu") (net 9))
 (segment (start 111.6165 91.5781) (end 113.7385 89.4561) (width 0.2) (layer "B.Cu") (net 9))
 (segment (start 107.2674 96.4489) (end 107.2674 93.2144) (width 0.2) (layer "B.Cu") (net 9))
 (segment (start 120.52 90.7025) (end 120.52 90.4611) (width 0.2) (layer "F.Cu") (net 5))
 (segment (start 114.0576 90.415) (end 111.115 90.415) (width 0.2) (layer "F.Cu") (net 5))
 (segment (start 119.2164 89.1575) (end 115.3151 89.1575) (width 0.2) (layer "F.Cu") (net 5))
 (segment (start 120.52 90.4611) (end 119.2164 89.1575) (width 0.2) (layer "F.Cu") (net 5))
 (segment (start 115.3151 89.1575) (end 114.0576 90.415) (width 0.2) (layer "F.Cu") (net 5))
 (segment (start 118.3065 89.5592) (end 119.25 90.5027) (width 0.2) (layer "F.Cu") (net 6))
 (segment (start 110.9475 92.7875) (end 109.1803 92.7875) (width 0.2) (layer "F.Cu") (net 6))
 (segment (start 108.8355 93.1323) (end 108.8355 94.4105) (width 0.2) (layer "F.Cu") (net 6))
 (segment (start 108.8355 94.4105) (end 109.615 95.19) (width 0.2) (layer "F.Cu") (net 6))
 (segment (start 115.9824 89.5592) (end 118.3065 89.5592) (width 0.2) (layer "F.Cu") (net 6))
 (segment (start 111.115 92.955) (end 110.9475 92.7875) (width 0.2) (layer "F.Cu") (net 6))
 (segment (start 109.1803 92.7875) (end 108.8355 93.1323) (width 0.2) (layer "F.Cu") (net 6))
 (segment (start 115.6696 89.872) (end 115.9824 89.5592) (width 0.2) (layer "F.Cu") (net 6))
 (segment (start 119.25 90.5027) (end 119.25 90.7025) (width 0.2) (layer "F.Cu") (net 6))
 (via (at 115.6696 89.872) (size 0.6) (drill 0.3) (layers "F.Cu" "B.Cu") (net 6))
 (segment (start 114.3172 89.872) (end 115.6696 89.872) (width 0.2) (layer "B.Cu") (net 6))
 (segment (start 111.2343 92.955) (end 111.2343 92.9549) (width 0.2) (layer "B.Cu") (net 6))
 (segment (start 111.2343 92.9549) (end 114.3172 89.872) (width 0.2) (layer "B.Cu") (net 6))
 (segment (start 111.115 92.955) (end 111.2343 92.955) (width 0.2) (layer "B.Cu") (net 6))
 (segment (start 115.6566 92.2697) (end 116.6753 92.2697) (width 0.2) (layer "F.Cu") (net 7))
 (segment (start 117.98 90.965) (end 117.98 90.7025) (width 0.2) (layer "F.Cu") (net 7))
 (segment (start 116.6753 92.2697) (end 117.98 90.965) (width 0.2) (layer "F.Cu") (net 7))
 (via (at 115.6566 92.2697) (size 0.6) (drill 0.3) (layers "F.Cu" "B.Cu") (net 7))
 (segment (start 113.7297 91.0276) (end 114.4145 91.0276) (width 0.2) (layer "B.Cu") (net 7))
 (segment (start 111.115 95.495) (end 112.9704 93.6396) (width 0.2) (layer "B.Cu") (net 7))
 (segment (start 112.9704 91.7869) (end 113.7297 91.0276) (width 0.2) (layer "B.Cu") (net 7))
 (segment (start 112.9704 93.6396) (end 112.9704 91.7869) (width 0.2) (layer "B.Cu") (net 7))
 (segment (start 114.4145 91.0276) (end 115.6566 92.2697) (width 0.2) (layer "B.Cu") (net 7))
 (segment (start 116.9941 99.0632) (end 116.3562 99.0632) (width 0.2) (layer "F.Cu") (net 2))
 (segment (start 117.3383 95.77) (end 125.615 95.77) (width 0.2) (layer "F.Cu") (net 2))
 (segment (start 116.0709 98.7779) (end 116.0709 97.0374) (width 0.2) (layer "F.Cu") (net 2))
 (segment (start 116.3562 99.0632) (end 116.0709 98.7779) (width 0.2) (layer "F.Cu") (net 2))
 (segment (start 110.3178 99.5428) (end 109.615 98.84) (width 0.2) (layer "F.Cu") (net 2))
 (segment (start 117.98 98.0773) (end 116.9941 99.0632) (width 0.2) (layer "F.Cu") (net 2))
 (segment (start 116.5145 99.5428) (end 110.3178 99.5428) (width 0.2) (layer "F.Cu") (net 2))
 (segment (start 117.98 97.8775) (end 117.98 98.0773) (width 0.2) (layer "F.Cu") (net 2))
 (segment (start 116.0709 97.0374) (end 117.3383 95.77) (width 0.2) (layer "F.Cu") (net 2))
 (segment (start 116.9941 99.0632) (end 116.5145 99.5428) (width 0.2) (layer "F.Cu") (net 2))
 (segment (start 125.615 93.23) (end 114.505 93.23) (width 0.2) (layer "F.Cu") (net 3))
 (segment (start 120.5165 96.3966) (end 124.0819 96.3966) (width 0.2) (layer "F.Cu") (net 3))
 (segment (start 126.112 96.9226) (end 126.8052 96.2294) (width 0.2) (layer "F.Cu") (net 3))
 (segment (start 119.25 97.6631) (end 120.5165 96.3966) (width 0.2) (layer "F.Cu") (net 3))
 (segment (start 124.0819 96.3966) (end 124.6079 96.9226) (width 0.2) (layer "F.Cu") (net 3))
 (segment (start 126.8052 96.2294) (end 126.8052 94.4202) (width 0.2) (layer "F.Cu") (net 3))
 (segment (start 126.8052 94.4202) (end 125.615 93.23) (width 0.2) (layer "F.Cu") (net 3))
 (segment (start 119.25 97.8775) (end 119.25 97.6631) (width 0.2) (layer "F.Cu") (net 3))
 (segment (start 124.6079 96.9226) (end 126.112 96.9226) (width 0.2) (layer "F.Cu") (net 3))
 (segment (start 114.505 93.23) (end 112.615 91.34) (width 0.2) (layer "F.Cu") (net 3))
 (segment (start 116.71 97.6413) (end 117.8884 96.4629) (width 0.2) (layer "F.Cu") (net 1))
 (segment (start 116.71 97.8775) (end 116.71 97.6413) (width 0.2) (layer "F.Cu") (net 1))
 (segment (start 117.8884 96.4629) (end 119.0371 96.4629) (width 0.2) (layer "F.Cu") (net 1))
 (via (at 119.0371 96.4629) (size 0.6) (drill 0.3) (layers "F.Cu" "B.Cu") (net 1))
 (segment (start 120.8842 98.31) (end 119.0371 96.4629) (width 0.2) (layer "B.Cu") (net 1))
 (segment (start 125.615 98.31) (end 120.8842 98.31) (width 0.2) (layer "B.Cu") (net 1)))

